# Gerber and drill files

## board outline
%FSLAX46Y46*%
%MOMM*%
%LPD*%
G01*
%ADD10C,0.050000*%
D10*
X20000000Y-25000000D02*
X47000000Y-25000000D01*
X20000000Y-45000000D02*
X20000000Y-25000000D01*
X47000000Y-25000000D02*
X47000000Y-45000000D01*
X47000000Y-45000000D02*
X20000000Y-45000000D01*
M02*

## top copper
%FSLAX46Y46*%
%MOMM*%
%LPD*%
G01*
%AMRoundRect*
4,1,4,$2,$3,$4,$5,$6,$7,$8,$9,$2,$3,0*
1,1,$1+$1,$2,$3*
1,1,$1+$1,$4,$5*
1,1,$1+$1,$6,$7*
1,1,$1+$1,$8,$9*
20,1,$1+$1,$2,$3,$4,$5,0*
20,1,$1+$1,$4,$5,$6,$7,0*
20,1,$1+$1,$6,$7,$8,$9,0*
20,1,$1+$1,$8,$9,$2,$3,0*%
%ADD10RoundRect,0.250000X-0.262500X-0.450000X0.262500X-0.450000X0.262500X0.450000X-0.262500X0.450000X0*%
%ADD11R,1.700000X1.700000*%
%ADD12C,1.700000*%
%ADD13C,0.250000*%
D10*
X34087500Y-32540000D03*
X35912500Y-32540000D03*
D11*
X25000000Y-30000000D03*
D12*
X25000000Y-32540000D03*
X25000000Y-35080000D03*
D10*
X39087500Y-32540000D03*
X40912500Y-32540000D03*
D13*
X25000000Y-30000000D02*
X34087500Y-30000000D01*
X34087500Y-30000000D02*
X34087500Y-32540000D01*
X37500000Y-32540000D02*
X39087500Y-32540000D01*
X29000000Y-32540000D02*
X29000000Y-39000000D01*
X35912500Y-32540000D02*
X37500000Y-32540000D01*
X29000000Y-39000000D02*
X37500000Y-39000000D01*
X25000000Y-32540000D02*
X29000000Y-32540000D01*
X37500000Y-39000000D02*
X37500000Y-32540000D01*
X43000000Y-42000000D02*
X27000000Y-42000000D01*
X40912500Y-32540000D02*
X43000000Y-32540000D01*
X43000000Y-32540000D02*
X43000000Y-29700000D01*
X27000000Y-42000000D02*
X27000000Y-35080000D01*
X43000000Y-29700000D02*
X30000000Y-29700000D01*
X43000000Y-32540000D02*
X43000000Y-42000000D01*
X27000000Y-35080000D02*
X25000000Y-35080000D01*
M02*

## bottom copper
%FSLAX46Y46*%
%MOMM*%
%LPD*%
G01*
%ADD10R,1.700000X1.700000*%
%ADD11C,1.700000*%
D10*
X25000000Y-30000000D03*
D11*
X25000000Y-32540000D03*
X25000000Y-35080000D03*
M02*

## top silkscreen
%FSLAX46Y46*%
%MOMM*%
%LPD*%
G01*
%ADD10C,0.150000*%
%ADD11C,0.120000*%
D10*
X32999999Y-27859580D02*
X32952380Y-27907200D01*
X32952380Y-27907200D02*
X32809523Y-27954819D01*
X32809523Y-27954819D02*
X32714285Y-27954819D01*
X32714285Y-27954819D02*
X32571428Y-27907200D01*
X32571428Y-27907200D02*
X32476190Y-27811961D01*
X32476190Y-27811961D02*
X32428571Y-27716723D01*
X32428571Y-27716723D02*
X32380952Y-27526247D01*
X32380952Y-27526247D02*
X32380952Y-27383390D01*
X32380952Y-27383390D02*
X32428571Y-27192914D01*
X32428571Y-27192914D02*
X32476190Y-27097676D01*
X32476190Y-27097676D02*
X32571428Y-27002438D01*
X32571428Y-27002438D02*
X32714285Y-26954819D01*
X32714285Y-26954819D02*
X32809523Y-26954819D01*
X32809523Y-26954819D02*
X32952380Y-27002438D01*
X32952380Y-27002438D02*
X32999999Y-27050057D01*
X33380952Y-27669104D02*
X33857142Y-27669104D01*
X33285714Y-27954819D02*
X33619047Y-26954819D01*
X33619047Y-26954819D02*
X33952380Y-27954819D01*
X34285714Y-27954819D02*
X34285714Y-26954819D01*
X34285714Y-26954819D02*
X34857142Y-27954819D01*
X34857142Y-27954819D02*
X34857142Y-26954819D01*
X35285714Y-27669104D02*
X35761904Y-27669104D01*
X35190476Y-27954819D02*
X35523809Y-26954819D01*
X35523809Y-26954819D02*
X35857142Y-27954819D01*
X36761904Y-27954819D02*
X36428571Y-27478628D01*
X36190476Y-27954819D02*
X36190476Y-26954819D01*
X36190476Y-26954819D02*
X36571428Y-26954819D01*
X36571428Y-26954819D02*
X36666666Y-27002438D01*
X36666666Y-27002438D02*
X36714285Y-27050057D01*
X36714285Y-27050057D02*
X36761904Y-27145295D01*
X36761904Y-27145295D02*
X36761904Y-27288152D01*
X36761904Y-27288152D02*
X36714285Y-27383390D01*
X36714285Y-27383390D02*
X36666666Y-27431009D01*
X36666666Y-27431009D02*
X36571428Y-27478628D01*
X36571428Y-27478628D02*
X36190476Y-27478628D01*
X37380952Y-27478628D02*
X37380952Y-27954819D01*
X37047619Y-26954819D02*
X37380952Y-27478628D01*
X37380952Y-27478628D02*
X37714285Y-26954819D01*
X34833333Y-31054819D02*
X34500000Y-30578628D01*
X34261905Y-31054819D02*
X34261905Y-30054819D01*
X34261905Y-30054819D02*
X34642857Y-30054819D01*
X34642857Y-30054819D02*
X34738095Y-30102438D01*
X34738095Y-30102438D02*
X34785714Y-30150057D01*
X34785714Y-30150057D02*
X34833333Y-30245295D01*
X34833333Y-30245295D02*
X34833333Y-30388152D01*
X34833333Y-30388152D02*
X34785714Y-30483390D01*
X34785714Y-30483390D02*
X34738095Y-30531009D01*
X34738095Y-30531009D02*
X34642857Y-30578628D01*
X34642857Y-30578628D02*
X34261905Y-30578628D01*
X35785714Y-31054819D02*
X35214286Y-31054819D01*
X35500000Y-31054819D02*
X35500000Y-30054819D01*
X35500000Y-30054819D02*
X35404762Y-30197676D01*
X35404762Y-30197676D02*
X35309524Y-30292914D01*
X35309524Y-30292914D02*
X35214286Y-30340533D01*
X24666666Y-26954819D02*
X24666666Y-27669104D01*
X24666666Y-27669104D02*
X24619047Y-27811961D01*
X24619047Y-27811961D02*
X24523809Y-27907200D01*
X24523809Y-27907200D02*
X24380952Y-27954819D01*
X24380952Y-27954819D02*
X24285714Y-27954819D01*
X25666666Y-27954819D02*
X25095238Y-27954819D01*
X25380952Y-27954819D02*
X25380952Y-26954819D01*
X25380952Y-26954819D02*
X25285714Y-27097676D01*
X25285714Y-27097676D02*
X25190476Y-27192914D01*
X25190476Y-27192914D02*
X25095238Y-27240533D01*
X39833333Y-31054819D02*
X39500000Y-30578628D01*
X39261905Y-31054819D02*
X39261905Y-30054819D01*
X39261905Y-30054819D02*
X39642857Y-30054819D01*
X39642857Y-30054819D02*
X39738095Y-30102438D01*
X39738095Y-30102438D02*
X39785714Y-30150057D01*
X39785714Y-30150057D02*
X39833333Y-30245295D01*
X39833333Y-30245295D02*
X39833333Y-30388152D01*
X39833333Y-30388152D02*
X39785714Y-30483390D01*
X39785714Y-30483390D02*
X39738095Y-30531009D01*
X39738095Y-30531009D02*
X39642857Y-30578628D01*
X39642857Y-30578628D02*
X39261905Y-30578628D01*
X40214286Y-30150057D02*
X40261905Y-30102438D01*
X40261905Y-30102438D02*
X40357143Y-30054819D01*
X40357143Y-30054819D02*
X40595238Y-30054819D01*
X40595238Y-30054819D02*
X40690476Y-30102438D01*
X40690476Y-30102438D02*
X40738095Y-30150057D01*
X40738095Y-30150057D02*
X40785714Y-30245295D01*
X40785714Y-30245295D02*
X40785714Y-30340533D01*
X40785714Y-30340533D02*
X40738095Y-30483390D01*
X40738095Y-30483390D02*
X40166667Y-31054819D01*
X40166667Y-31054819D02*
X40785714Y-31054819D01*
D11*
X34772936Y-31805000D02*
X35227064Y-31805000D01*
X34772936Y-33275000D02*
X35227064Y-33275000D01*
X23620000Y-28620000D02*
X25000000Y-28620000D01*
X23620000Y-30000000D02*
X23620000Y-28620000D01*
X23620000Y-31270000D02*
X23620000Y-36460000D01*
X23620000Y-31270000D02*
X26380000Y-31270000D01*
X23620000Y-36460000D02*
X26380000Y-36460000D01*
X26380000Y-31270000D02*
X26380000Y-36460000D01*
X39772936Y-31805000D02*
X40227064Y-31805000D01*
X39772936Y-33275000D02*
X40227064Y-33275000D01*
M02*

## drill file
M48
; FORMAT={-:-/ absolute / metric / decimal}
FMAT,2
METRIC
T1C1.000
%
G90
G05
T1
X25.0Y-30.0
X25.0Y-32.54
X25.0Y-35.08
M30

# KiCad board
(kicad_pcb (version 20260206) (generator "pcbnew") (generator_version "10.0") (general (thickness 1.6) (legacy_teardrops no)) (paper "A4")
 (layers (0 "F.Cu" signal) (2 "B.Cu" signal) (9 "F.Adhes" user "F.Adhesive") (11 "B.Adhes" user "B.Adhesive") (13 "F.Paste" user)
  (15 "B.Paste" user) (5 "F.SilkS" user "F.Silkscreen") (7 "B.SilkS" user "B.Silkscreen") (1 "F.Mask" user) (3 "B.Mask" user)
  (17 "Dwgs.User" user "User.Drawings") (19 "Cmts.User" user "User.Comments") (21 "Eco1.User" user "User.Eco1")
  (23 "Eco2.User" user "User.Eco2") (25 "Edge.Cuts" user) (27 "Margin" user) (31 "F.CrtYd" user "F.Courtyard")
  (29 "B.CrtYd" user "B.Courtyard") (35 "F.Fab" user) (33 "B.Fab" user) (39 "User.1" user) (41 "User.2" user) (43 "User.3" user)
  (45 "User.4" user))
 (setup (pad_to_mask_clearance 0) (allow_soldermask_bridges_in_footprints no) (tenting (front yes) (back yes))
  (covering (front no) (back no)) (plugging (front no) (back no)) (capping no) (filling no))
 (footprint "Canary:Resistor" (layer "F.Cu") (at 35 32.54)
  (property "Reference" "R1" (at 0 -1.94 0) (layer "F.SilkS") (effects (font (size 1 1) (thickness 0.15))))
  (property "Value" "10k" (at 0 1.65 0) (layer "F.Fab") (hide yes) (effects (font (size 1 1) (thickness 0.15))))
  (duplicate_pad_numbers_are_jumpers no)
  (fp_line (start -0.227064 -0.735) (end 0.227064 -0.735) (stroke (width 0.12) (type solid)) (layer "F.SilkS"))
  (fp_line (start -0.227064 0.735) (end 0.227064 0.735) (stroke (width 0.12) (type solid)) (layer "F.SilkS"))
  (pad "1" smd roundrect (at -0.9125 0) (size 1.025 1.4) (layers "F.Cu" "F.Mask" "F.Paste") (roundrect_rratio 0.243902) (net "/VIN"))
  (pad "2" smd roundrect (at 0.9125 0) (size 1.025 1.4) (layers "F.Cu" "F.Mask" "F.Paste") (roundrect_rratio 0.243902) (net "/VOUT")))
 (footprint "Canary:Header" (layer "F.Cu") (at 25 30)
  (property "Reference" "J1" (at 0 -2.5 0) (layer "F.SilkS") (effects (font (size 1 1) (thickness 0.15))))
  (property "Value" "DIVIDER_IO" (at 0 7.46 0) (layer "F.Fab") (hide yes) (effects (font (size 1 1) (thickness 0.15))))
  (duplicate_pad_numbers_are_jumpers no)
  (fp_line (start -1.38 -1.38) (end 0 -1.38) (stroke (width 0.12) (type solid)) (layer "F.SilkS"))
  (fp_line (start -1.38 0) (end -1.38 -1.38) (stroke (width 0.12) (type solid)) (layer "F.SilkS"))
  (fp_line (start -1.38 1.27) (end -1.38 6.46) (stroke (width 0.12) (type solid)) (layer "F.SilkS"))
  (fp_line (start -1.38 1.27) (end 1.38 1.27) (stroke (width 0.12) (type solid)) (layer "F.SilkS"))
  (fp_line (start -1.38 6.46) (end 1.38 6.46) (stroke (width 0.12) (type solid)) (layer "F.SilkS"))
  (fp_line (start 1.38 1.27) (end 1.38 6.46) (stroke (width 0.12) (type solid)) (layer "F.SilkS"))
  (pad "1" thru_hole rect (at 0 0) (size 1.7 1.7) (drill 1) (layers "*.Cu" "*.Mask") (remove_unused_layers no) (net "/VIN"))
  (pad "2" thru_hole circle (at 0 2.54) (size 1.7 1.7) (drill 1) (layers "*.Cu" "*.Mask") (remove_unused_layers no) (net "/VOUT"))
  (pad "3" thru_hole circle (at 0 5.08) (size 1.7 1.7) (drill 1) (layers "*.Cu" "*.Mask") (remove_unused_layers no) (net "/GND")))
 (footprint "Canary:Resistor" (layer "F.Cu") (at 40 32.54)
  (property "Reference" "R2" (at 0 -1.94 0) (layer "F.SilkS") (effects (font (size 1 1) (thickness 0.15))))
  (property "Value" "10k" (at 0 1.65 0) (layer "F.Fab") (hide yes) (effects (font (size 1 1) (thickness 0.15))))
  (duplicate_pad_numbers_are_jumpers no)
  (fp_line (start -0.227064 -0.735) (end 0.227064 -0.735) (stroke (width 0.12) (type solid)) (layer "F.SilkS"))
  (fp_line (start -0.227064 0.735) (end 0.227064 0.735) (stroke (width 0.12) (type solid)) (layer "F.SilkS"))
  (pad "1" smd roundrect (at -0.9125 0) (size 1.025 1.4) (layers "F.Cu" "F.Mask" "F.Paste") (roundrect_rratio 0.243902) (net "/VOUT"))
  (pad "2" smd roundrect (at 0.9125 0) (size 1.025 1.4) (layers "F.Cu" "F.Mask" "F.Paste") (roundrect_rratio 0.243902) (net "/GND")))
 (gr_line (start 20 25) (end 47 25) (stroke (width 0.05) (type default)) (layer "Edge.Cuts"))
 (gr_line (start 20 45) (end 20 25) (stroke (width 0.05) (type default)) (layer "Edge.Cuts"))
 (gr_line (start 47 25) (end 47 45) (stroke (width 0.05) (type default)) (layer "Edge.Cuts"))
 (gr_line (start 47 45) (end 20 45) (stroke (width 0.05) (type default)) (layer "Edge.Cuts"))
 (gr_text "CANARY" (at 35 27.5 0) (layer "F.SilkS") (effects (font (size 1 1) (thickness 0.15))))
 (segment (start 25 30) (end 34.0875 30) (width 0.25) (layer "F.Cu") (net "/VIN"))
 (segment (start 34.0875 30) (end 34.0875 32.54) (width 0.25) (layer "F.Cu") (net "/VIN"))
 (segment (start 37.5 32.54) (end 39.0875 32.54) (width 0.25) (layer "F.Cu") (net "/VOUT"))
 (segment (start 29 32.54) (end 29 39) (width 0.25) (layer "F.Cu") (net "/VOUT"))
 (segment (start 35.9125 32.54) (end 37.5 32.54) (width 0.25) (layer "F.Cu") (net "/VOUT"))
 (segment (start 29 39) (end 37.5 39) (width 0.25) (layer "F.Cu") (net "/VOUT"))
 (segment (start 25 32.54) (end 29 32.54) (width 0.25) (layer "F.Cu") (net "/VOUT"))
 (segment (start 37.5 39) (end 37.5 32.54) (width 0.25) (layer "F.Cu") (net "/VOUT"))
 (segment (start 43 42) (end 27 42) (width 0.25) (layer "F.Cu") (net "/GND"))
 (segment (start 40.9125 32.54) (end 43 32.54) (width 0.25) (layer "F.Cu") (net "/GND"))
 (segment (start 43 32.54) (end 43 29.7) (width 0.25) (layer "F.Cu") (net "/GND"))
 (segment (start 27 42) (end 27 35.08) (width 0.25) (layer "F.Cu") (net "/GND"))
 (segment (start 43 29.7) (end 30 29.7) (width 0.25) (layer "F.Cu") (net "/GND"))
 (segment (start 43 32.54) (end 43 42) (width 0.25) (layer "F.Cu") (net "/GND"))
 (segment (start 27 35.08) (end 25 35.08) (width 0.25) (layer "F.Cu") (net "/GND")))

